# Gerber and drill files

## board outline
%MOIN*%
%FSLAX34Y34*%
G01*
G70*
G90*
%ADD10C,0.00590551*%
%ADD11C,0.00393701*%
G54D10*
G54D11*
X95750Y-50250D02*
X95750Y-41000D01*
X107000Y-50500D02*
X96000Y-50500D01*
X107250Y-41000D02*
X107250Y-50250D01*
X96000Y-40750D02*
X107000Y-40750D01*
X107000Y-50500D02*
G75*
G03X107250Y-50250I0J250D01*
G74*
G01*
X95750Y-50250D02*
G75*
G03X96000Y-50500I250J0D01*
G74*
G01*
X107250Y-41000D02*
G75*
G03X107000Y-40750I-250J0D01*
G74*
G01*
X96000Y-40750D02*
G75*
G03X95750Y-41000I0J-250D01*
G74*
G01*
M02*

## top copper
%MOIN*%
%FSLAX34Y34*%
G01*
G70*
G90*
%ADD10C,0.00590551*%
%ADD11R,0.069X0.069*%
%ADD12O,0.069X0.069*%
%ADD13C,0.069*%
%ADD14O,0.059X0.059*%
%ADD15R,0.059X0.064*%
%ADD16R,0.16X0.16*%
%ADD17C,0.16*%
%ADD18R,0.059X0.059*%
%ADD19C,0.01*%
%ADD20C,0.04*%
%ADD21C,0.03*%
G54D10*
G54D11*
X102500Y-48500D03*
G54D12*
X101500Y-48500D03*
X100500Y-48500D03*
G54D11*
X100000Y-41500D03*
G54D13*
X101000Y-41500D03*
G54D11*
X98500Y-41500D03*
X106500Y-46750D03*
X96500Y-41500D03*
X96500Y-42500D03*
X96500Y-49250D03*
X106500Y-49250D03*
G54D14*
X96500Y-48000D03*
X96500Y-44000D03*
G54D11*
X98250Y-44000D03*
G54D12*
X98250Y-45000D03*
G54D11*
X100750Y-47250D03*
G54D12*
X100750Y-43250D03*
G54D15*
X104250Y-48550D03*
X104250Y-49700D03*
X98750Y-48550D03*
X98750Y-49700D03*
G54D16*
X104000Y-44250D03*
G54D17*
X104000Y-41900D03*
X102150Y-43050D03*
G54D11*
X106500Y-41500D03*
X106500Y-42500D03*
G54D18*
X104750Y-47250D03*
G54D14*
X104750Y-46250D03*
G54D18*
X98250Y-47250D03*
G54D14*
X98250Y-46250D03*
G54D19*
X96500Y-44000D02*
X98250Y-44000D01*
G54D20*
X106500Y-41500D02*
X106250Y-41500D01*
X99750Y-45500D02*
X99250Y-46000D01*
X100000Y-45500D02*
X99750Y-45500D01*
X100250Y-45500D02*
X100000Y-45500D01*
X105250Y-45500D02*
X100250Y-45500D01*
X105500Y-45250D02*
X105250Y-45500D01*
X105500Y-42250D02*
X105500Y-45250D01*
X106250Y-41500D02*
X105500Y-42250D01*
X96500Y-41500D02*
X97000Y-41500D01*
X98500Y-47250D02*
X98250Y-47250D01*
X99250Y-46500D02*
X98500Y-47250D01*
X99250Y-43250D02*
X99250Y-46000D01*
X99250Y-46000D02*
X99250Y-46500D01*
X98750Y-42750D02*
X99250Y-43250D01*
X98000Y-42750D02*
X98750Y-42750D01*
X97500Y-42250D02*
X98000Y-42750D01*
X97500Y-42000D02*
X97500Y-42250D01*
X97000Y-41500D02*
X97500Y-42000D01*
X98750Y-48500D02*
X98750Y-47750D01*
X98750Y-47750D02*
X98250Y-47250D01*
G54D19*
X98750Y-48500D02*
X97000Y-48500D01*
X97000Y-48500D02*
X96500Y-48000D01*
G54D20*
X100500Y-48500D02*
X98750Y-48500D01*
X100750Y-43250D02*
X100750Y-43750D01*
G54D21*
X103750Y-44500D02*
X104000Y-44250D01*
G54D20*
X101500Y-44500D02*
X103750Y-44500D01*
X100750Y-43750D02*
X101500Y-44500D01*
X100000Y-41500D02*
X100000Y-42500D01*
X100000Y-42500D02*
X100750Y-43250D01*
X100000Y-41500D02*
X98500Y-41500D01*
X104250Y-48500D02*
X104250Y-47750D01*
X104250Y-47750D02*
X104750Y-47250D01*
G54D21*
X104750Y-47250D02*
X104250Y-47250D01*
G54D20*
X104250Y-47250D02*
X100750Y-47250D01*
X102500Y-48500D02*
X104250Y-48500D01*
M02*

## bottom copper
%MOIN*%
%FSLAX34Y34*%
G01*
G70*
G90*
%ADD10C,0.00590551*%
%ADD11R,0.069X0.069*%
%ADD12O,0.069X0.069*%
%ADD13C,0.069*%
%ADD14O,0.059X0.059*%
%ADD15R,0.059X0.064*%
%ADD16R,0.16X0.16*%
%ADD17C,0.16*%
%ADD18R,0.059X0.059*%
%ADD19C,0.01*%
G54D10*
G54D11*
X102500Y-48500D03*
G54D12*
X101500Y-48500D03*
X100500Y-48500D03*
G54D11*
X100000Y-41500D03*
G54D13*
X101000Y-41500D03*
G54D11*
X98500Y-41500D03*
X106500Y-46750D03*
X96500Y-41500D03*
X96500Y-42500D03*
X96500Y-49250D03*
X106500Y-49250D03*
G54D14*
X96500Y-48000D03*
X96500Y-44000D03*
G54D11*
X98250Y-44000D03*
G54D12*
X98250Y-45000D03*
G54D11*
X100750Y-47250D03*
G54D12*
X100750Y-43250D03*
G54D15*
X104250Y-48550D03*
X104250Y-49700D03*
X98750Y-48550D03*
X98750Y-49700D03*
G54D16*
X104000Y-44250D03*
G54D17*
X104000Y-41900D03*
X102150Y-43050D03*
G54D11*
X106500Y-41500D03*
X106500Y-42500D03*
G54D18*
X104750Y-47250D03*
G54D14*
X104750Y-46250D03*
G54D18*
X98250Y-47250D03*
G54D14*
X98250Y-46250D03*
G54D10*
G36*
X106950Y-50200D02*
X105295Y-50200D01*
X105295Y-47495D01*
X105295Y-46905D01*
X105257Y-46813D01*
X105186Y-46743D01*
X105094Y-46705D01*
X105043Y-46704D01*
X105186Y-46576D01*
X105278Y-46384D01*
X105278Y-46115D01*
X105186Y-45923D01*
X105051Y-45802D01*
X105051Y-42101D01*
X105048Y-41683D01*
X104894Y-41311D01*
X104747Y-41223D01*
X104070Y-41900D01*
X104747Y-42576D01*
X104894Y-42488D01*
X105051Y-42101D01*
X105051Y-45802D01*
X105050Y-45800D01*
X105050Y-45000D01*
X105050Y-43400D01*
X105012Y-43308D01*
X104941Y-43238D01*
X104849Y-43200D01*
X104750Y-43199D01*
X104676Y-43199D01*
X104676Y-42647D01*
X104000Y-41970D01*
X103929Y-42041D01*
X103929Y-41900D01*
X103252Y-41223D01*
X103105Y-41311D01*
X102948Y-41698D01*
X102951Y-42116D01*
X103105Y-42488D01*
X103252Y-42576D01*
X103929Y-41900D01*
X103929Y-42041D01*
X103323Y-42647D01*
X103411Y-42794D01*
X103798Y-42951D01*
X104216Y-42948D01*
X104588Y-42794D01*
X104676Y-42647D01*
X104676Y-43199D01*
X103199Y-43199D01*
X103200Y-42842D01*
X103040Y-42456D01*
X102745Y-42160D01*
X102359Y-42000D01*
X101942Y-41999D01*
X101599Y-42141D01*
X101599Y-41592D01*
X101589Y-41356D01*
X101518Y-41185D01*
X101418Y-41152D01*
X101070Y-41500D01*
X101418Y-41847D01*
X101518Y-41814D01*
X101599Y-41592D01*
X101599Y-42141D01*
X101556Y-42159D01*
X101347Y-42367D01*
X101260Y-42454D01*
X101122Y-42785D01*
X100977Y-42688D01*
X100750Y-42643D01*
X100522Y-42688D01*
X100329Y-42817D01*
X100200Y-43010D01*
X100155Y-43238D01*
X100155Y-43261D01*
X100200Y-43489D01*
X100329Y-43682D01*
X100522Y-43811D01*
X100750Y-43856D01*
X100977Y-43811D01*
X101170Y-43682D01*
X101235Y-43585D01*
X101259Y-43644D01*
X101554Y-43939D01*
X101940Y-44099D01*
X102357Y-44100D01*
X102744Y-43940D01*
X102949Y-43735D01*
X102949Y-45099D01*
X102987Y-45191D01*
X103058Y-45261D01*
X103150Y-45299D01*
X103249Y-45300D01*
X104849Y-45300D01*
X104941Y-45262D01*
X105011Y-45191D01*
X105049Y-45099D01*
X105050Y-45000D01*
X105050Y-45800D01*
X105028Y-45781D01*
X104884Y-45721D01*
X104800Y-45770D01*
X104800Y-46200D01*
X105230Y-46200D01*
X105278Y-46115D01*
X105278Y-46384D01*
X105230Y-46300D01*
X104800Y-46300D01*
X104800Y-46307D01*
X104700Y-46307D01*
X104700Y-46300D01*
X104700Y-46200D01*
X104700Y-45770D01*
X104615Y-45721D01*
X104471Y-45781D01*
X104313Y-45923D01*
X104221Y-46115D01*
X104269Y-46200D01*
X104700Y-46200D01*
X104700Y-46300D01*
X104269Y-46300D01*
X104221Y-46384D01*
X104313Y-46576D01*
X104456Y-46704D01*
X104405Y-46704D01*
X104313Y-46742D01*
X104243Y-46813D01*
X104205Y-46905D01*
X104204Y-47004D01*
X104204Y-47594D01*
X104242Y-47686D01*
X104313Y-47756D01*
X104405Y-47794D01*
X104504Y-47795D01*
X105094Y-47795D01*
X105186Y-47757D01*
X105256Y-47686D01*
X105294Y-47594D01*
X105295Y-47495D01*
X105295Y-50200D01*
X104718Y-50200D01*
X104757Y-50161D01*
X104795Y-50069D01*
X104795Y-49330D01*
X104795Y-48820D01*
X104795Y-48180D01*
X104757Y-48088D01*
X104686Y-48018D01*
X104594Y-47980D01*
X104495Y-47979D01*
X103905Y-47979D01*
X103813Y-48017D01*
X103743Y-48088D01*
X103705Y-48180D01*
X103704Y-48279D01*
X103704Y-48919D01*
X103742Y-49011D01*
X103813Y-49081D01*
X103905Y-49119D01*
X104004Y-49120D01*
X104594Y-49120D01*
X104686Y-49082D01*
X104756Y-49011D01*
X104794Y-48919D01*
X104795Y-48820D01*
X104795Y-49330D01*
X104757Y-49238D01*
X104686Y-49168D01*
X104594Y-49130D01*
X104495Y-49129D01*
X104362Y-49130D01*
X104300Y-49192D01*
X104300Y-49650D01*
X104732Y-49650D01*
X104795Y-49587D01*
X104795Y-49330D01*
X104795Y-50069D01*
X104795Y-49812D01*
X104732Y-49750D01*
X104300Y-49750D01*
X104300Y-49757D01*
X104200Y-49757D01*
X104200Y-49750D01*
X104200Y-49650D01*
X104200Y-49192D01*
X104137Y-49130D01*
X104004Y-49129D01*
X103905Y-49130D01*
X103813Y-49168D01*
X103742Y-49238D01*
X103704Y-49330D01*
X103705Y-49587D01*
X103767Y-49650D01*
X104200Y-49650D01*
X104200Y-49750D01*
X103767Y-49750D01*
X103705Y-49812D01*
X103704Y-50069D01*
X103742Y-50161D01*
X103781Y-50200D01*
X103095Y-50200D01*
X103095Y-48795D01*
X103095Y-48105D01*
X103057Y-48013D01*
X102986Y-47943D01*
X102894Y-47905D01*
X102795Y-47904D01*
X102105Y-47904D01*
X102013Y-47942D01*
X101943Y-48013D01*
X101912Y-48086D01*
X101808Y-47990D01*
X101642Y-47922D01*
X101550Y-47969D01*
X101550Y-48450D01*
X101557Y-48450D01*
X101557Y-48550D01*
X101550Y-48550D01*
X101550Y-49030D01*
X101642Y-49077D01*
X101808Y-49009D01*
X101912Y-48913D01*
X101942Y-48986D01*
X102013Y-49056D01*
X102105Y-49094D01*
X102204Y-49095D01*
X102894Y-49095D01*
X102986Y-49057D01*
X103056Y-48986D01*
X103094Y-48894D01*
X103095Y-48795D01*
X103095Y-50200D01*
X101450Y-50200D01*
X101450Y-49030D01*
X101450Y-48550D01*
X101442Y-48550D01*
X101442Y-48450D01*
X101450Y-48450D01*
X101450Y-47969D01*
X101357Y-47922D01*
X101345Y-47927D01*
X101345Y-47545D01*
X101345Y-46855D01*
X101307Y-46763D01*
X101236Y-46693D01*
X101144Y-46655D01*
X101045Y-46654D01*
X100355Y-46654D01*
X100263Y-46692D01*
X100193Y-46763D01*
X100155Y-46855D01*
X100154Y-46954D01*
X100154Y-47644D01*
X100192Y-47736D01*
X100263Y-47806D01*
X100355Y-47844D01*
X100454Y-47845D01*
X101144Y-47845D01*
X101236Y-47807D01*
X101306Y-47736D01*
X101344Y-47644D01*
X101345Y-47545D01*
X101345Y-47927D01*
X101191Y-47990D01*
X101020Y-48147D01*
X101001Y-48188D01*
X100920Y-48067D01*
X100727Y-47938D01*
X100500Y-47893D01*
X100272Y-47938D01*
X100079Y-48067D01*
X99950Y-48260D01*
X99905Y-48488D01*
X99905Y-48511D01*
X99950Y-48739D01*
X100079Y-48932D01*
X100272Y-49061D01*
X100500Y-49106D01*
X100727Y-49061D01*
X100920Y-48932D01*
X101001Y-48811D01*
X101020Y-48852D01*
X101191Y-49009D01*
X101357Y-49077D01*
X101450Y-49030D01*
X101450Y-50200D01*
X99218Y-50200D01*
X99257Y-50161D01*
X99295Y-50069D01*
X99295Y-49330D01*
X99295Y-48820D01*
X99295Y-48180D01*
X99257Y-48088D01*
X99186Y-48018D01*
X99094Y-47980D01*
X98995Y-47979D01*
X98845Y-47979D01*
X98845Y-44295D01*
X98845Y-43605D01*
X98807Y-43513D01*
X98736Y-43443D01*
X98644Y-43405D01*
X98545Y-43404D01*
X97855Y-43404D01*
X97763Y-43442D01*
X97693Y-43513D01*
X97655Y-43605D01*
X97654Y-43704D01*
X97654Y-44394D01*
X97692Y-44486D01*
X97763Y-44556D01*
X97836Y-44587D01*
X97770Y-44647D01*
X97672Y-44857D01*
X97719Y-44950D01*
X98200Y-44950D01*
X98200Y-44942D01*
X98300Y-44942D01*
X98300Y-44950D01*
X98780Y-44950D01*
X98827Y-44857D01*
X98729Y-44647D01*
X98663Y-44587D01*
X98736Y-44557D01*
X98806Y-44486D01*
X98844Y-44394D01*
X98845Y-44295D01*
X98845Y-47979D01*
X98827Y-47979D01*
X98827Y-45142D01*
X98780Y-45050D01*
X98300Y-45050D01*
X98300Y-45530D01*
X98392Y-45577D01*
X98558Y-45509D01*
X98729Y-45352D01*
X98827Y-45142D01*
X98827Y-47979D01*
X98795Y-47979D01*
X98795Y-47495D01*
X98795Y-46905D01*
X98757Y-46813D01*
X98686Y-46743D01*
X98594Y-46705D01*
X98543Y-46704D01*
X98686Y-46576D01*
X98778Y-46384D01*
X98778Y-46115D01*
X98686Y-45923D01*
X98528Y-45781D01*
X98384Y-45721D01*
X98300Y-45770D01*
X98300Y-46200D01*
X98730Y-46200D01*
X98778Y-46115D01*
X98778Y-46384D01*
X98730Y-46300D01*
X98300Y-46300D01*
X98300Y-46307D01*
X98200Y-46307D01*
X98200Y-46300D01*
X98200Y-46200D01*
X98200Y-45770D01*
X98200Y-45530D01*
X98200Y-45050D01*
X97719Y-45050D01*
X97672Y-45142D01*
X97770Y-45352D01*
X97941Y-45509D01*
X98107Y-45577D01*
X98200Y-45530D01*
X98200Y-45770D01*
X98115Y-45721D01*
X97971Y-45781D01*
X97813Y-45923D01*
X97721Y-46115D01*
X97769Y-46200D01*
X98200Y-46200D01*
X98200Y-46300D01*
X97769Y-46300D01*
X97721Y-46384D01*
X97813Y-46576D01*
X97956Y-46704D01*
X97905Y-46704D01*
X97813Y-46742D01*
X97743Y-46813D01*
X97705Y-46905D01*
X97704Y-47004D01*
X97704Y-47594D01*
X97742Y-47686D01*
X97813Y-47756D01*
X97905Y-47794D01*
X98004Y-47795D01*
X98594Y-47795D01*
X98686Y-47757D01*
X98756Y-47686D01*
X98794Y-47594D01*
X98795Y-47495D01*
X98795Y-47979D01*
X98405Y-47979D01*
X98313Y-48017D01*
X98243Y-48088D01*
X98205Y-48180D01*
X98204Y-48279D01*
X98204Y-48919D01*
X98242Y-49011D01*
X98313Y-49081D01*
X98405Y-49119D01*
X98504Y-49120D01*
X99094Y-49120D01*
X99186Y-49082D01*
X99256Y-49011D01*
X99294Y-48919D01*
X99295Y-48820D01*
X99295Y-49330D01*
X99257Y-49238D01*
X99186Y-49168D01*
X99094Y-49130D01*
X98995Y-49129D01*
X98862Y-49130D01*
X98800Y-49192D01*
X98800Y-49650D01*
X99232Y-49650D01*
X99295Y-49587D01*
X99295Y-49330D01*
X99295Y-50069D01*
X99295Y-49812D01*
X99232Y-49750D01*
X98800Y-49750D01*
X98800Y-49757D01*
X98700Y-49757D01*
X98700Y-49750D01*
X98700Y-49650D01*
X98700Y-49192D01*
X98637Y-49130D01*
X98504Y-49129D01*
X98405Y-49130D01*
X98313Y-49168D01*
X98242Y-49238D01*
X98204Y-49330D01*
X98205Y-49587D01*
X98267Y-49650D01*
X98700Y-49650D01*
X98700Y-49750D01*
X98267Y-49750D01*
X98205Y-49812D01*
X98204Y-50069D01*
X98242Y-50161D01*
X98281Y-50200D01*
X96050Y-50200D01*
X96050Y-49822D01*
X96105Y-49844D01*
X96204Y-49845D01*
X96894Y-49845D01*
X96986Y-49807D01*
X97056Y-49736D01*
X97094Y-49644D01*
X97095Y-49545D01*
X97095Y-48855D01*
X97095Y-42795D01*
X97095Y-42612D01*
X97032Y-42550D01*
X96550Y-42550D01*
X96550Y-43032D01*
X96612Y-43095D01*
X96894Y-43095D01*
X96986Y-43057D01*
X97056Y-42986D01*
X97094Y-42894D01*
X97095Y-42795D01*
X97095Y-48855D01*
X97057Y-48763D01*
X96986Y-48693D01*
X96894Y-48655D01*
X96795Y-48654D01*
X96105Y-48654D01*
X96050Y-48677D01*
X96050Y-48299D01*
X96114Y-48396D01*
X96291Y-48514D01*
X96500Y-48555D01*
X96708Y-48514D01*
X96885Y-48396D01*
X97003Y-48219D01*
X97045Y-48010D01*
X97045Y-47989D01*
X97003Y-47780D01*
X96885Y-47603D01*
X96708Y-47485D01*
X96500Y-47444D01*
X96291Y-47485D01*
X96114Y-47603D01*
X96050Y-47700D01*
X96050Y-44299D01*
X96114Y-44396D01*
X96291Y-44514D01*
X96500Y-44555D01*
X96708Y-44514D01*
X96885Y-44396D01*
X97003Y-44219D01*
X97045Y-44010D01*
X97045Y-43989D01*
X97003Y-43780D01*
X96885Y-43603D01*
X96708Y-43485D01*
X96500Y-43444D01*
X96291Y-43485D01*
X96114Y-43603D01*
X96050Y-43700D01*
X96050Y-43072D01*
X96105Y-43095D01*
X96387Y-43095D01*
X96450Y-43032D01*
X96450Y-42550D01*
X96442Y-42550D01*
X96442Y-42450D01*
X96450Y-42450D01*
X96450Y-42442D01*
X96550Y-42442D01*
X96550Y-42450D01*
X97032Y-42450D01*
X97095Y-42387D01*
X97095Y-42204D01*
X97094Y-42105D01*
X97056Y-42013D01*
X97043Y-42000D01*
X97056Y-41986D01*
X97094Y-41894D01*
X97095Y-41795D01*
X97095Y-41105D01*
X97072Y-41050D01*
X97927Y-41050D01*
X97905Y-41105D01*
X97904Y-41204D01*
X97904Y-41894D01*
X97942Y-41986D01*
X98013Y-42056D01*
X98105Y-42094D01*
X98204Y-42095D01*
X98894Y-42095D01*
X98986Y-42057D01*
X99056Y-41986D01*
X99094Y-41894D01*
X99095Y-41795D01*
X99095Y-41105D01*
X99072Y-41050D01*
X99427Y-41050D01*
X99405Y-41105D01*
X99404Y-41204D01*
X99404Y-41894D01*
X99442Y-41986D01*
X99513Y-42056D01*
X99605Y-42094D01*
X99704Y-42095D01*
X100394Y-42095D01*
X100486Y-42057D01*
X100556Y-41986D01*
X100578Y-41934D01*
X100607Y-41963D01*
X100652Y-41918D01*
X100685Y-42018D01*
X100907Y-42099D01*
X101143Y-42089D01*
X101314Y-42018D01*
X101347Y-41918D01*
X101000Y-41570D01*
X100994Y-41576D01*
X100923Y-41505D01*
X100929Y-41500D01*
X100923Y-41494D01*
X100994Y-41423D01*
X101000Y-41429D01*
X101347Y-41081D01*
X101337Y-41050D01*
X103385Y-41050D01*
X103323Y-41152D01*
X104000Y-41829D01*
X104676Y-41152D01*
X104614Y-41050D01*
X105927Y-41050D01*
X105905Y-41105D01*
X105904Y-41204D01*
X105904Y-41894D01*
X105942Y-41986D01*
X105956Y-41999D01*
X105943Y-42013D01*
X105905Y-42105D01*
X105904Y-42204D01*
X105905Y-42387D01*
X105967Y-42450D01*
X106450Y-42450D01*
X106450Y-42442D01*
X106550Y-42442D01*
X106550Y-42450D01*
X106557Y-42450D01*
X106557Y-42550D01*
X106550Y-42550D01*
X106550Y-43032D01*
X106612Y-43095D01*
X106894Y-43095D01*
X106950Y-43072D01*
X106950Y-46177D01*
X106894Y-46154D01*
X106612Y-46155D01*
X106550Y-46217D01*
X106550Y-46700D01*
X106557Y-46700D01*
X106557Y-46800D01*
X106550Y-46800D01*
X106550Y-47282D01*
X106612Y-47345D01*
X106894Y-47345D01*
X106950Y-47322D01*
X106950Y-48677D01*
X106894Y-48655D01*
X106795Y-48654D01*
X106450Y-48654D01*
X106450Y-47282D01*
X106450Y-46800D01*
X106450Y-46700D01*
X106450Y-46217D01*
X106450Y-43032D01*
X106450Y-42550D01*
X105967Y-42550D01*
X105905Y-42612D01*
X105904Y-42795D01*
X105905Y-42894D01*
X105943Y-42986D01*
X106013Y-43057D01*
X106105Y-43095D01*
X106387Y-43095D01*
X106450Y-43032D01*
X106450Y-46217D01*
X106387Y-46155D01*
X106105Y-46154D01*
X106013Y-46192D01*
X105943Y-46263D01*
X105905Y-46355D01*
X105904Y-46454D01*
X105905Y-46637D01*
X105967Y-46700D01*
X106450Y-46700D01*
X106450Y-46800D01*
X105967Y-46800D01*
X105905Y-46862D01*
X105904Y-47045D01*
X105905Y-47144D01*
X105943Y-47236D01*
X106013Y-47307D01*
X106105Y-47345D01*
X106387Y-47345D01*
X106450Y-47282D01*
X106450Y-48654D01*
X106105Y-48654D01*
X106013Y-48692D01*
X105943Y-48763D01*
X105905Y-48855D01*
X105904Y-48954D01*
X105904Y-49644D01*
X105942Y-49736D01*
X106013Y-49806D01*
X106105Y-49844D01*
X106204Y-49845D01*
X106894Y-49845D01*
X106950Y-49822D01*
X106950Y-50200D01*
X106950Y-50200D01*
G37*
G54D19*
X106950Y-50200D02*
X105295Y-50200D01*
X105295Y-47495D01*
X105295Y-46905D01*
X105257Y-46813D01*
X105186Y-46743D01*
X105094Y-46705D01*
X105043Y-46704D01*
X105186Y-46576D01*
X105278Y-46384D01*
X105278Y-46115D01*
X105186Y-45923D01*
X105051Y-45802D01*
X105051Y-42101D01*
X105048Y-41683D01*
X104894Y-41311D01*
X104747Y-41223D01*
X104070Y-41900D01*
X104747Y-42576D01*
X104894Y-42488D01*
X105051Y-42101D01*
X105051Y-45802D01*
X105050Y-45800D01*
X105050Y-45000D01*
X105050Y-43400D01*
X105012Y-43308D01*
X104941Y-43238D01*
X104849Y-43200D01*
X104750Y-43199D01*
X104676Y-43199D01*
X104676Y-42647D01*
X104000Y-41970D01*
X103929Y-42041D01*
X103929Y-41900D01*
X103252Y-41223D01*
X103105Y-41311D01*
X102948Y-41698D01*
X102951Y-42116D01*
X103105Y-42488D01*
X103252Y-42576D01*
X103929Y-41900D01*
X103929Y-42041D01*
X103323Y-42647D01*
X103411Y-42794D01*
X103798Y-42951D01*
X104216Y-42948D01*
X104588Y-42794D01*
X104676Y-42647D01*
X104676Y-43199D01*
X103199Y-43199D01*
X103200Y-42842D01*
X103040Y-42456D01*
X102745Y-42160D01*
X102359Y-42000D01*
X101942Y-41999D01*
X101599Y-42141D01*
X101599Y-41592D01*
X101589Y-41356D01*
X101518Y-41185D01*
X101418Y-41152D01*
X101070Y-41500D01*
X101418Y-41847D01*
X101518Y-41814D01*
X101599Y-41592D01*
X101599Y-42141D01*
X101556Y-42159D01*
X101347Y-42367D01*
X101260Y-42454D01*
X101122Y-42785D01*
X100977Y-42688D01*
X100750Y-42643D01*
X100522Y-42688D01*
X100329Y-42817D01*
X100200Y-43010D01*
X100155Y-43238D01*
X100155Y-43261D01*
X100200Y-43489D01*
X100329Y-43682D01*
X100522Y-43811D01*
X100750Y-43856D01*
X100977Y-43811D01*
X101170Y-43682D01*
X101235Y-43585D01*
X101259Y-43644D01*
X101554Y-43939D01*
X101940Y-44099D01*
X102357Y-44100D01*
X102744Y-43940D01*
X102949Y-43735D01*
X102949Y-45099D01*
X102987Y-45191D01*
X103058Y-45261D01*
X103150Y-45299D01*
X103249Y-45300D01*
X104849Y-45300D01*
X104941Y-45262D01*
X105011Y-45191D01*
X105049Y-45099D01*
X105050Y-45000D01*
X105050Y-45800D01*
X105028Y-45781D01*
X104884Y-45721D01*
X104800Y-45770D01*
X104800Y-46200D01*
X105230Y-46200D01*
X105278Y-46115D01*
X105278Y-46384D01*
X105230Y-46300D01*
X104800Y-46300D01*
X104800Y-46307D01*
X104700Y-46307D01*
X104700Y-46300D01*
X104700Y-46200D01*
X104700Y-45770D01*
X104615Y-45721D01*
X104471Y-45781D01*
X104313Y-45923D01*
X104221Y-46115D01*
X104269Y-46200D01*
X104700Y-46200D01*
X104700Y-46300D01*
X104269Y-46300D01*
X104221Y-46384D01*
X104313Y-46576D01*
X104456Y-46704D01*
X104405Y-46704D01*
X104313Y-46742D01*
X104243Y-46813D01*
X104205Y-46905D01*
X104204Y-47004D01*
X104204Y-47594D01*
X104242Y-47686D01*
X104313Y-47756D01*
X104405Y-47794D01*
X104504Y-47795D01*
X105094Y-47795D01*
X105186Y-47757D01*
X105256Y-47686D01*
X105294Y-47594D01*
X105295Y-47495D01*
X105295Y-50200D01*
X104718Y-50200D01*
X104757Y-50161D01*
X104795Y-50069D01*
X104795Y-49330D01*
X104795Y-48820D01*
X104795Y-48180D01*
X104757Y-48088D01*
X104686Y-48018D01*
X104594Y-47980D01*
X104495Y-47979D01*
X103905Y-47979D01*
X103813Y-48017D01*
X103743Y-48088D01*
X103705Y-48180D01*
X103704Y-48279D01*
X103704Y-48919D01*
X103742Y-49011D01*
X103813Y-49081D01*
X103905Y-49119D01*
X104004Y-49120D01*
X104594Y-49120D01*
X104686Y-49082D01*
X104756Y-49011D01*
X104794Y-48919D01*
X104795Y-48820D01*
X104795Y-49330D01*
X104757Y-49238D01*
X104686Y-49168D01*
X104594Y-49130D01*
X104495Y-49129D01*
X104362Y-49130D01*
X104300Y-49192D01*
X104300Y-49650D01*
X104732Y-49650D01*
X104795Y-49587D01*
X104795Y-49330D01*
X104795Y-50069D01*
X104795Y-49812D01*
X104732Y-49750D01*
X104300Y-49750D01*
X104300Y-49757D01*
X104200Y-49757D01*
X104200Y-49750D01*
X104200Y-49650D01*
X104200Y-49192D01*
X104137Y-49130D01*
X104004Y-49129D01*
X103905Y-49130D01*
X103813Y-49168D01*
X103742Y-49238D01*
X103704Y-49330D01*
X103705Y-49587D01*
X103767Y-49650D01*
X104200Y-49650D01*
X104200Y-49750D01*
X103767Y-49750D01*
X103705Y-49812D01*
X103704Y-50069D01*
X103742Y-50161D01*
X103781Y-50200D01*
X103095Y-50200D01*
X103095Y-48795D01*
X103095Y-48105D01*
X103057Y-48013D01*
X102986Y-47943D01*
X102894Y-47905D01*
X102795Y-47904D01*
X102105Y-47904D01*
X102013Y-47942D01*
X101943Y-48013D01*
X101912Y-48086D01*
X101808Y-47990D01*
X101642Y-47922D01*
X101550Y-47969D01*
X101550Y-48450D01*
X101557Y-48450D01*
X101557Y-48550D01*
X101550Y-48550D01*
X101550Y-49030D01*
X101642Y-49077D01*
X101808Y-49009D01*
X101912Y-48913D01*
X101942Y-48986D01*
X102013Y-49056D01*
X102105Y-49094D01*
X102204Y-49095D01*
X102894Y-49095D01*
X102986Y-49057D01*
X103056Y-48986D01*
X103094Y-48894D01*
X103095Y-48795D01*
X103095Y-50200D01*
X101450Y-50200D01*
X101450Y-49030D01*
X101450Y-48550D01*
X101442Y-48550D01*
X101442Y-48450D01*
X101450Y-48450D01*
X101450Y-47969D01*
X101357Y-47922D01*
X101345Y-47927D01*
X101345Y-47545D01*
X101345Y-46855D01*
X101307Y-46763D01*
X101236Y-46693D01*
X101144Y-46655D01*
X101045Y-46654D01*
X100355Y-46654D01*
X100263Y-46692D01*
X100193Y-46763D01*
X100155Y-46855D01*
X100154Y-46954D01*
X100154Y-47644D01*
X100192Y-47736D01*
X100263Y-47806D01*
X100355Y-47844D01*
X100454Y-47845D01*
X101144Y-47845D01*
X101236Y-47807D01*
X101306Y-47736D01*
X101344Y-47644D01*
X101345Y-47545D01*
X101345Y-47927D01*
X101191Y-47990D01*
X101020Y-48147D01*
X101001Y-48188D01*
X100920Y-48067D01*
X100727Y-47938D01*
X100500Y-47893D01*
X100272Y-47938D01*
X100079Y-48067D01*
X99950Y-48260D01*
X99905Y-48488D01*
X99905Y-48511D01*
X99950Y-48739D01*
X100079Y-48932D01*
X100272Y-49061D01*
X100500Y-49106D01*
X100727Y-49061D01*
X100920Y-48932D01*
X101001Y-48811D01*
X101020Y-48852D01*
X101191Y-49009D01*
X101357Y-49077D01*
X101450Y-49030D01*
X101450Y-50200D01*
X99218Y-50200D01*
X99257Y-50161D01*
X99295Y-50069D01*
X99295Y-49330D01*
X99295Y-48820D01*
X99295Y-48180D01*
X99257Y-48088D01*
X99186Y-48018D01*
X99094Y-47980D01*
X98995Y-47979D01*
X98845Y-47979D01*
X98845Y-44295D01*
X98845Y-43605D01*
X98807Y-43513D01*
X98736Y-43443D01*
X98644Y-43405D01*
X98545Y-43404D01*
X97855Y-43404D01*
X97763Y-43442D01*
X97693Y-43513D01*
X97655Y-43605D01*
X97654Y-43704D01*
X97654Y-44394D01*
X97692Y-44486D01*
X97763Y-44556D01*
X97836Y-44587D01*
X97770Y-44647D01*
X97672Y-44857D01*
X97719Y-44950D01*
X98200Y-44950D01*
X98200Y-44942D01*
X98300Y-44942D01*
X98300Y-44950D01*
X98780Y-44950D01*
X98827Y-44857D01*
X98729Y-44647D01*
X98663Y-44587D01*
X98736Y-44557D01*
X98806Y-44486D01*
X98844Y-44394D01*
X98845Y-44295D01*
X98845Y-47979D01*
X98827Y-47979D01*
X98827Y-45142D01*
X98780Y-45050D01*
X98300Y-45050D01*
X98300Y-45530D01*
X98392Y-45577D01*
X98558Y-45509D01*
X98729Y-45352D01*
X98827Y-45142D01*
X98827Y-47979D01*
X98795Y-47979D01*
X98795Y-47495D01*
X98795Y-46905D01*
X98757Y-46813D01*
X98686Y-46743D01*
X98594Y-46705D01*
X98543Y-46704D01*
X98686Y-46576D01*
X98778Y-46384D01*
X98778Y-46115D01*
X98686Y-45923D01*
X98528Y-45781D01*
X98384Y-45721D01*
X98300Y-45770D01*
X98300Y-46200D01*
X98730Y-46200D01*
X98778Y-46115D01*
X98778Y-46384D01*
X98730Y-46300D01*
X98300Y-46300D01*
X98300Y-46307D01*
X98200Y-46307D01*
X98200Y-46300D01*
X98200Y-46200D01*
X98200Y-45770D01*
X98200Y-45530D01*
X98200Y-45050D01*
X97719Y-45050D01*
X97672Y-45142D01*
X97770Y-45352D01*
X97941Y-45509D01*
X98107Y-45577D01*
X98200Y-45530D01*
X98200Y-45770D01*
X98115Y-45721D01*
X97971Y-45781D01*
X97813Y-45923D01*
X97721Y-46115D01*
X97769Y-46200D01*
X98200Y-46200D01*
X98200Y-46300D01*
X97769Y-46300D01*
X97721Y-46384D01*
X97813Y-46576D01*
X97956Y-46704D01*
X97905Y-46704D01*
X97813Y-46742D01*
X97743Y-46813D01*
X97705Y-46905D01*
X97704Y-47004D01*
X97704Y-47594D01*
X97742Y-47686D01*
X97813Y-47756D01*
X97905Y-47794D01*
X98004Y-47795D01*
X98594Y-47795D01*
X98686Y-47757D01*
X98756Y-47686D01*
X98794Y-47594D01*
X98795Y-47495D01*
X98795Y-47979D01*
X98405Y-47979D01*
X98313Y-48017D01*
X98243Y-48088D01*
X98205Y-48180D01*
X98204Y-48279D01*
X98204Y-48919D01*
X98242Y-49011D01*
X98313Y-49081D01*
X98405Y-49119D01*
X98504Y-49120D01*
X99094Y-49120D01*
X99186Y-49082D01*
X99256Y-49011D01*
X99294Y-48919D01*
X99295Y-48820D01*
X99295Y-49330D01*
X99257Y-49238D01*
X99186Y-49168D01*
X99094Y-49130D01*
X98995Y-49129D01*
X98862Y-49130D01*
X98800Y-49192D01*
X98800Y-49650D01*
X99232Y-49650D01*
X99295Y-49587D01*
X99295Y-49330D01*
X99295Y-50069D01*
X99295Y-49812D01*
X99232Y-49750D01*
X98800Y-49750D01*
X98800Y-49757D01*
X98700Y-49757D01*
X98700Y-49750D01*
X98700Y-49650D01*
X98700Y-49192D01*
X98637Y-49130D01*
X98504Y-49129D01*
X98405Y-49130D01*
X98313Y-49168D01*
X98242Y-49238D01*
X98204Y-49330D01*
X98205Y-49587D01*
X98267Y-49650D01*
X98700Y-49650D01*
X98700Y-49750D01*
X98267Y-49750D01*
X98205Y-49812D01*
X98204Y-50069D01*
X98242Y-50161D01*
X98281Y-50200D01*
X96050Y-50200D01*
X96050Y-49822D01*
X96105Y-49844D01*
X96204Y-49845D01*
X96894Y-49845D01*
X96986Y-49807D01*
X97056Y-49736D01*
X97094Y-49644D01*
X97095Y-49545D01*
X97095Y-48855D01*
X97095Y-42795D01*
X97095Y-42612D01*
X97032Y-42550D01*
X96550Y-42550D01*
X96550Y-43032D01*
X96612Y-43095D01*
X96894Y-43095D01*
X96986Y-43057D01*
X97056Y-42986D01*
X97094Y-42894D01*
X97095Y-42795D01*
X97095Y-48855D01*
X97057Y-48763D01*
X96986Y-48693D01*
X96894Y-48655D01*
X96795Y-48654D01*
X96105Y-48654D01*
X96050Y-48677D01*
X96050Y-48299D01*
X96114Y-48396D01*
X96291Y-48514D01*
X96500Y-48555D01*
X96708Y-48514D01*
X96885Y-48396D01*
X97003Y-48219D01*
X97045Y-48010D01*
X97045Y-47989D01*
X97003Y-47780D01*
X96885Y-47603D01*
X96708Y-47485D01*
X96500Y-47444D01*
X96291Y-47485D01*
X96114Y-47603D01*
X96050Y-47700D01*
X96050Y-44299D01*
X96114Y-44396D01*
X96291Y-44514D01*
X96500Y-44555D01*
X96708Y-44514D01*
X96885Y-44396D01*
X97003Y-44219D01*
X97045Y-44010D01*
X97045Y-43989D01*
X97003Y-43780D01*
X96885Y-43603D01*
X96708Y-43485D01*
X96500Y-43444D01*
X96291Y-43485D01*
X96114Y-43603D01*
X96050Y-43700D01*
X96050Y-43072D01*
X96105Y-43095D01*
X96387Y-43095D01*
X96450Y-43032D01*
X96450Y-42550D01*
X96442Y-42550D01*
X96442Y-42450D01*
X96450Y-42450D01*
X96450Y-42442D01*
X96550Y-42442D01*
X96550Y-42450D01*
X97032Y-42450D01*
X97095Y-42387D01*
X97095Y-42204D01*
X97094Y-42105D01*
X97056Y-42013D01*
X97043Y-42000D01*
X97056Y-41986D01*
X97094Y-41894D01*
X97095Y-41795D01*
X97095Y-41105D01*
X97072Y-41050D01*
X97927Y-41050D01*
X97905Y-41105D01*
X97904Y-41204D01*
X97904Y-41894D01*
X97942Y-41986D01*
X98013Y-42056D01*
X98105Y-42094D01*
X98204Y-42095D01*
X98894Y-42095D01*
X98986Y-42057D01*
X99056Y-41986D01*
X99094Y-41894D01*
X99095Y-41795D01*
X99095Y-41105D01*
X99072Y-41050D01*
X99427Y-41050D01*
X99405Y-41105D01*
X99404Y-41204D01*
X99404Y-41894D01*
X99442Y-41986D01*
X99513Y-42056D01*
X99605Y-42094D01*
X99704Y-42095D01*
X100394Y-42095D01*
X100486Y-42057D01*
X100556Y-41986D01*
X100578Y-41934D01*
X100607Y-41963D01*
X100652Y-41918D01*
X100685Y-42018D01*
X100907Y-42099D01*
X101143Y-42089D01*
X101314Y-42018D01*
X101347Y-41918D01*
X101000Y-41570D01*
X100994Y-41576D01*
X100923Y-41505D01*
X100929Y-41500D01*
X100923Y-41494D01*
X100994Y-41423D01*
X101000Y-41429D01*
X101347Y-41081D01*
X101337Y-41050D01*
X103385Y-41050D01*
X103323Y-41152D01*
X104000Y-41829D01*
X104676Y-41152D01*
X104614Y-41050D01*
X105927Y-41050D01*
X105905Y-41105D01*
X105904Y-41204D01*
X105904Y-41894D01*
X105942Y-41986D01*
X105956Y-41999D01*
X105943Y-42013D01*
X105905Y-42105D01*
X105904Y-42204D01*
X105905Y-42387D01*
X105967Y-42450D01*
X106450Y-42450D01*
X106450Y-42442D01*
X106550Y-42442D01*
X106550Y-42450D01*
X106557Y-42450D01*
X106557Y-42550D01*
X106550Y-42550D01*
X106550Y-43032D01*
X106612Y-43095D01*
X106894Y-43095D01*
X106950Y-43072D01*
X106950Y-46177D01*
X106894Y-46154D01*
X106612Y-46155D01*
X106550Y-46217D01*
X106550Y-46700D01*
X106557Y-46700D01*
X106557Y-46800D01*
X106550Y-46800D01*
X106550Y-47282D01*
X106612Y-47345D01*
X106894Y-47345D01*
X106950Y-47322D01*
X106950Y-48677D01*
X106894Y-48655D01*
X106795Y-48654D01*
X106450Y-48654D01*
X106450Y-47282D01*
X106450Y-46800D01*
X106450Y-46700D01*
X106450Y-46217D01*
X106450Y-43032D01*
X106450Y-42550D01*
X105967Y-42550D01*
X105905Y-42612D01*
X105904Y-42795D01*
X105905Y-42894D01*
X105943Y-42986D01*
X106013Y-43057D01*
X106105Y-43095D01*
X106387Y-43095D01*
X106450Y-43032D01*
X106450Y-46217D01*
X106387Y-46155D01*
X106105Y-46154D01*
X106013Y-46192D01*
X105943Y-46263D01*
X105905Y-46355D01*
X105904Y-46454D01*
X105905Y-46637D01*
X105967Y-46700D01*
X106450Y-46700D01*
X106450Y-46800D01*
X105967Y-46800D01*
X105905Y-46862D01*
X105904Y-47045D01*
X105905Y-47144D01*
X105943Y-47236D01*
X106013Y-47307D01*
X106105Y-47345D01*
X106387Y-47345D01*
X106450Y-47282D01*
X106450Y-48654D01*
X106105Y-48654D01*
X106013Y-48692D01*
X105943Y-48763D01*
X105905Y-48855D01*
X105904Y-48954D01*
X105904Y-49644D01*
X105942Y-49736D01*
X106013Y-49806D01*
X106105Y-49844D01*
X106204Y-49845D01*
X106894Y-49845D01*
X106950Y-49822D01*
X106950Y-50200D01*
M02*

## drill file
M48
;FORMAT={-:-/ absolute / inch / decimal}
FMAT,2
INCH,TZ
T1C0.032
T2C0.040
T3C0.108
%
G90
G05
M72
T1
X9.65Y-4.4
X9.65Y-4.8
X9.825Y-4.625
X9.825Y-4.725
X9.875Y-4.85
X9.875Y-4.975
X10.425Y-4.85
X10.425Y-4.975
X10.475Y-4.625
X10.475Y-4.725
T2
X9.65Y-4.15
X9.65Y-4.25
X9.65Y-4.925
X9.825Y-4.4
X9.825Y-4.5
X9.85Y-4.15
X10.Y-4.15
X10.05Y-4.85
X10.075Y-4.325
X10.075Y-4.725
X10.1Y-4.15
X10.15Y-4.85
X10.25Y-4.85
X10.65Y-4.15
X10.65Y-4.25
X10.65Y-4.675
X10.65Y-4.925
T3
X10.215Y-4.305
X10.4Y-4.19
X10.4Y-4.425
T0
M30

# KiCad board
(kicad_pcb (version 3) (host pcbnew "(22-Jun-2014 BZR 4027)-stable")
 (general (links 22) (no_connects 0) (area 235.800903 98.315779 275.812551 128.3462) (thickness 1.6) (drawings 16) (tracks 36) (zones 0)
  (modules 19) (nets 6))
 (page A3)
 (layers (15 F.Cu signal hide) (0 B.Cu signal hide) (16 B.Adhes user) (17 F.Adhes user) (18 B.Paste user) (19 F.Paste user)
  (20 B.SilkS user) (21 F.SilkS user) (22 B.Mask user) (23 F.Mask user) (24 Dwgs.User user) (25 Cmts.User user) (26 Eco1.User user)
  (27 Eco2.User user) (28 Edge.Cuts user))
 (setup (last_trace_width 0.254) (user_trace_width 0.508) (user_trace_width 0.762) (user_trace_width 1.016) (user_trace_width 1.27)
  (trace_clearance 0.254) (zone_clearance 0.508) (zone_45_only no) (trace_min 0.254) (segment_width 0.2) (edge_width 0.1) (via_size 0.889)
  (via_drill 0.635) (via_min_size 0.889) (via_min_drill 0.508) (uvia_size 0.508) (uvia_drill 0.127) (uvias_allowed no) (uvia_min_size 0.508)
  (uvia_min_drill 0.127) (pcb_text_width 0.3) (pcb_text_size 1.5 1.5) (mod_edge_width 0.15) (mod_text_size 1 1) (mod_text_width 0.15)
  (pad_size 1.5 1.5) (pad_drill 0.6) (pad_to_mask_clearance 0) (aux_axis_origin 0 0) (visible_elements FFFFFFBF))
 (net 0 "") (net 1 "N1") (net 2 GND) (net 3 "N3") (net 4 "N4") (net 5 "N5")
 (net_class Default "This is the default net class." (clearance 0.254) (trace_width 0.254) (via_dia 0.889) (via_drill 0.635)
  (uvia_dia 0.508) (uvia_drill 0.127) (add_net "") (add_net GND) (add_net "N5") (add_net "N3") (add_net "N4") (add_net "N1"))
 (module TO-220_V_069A (layer F.Cu) (at 260.35 123.19 180)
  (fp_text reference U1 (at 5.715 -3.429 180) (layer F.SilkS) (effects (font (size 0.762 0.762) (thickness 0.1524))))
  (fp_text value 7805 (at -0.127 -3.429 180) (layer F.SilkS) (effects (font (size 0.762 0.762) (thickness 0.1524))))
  (pad 1 thru_hole rect (at 0 0 270) (size 1.7526 1.7526) (drill 1.016) (layers *.Cu *.Mask F.SilkS) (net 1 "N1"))
  (pad 2 thru_hole oval (at 2.54 0 270) (size 1.7526 1.7526) (drill 1.016) (layers *.Cu *.Mask F.SilkS) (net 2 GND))
  (pad 3 thru_hole oval (at 5.08 0 270) (size 1.7526 1.7526) (drill 1.016) (layers *.Cu *.Mask F.SilkS) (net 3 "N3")))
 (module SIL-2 (layer F.Cu) (at 254 105.41)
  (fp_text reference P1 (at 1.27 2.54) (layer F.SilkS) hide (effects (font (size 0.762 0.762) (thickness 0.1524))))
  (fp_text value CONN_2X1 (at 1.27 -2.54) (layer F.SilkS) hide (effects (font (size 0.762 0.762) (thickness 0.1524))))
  (pad 1 thru_hole rect (at 0 0) (size 1.7526 1.7526) (drill 1.016) (layers *.Cu *.Mask F.SilkS) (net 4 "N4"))
  (pad 2 thru_hole circle (at 2.54 0) (size 1.7526 1.7526) (drill 1.016) (layers *.Cu *.Mask F.SilkS) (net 2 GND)))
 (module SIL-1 (layer F.Cu) (at 250.19 105.41)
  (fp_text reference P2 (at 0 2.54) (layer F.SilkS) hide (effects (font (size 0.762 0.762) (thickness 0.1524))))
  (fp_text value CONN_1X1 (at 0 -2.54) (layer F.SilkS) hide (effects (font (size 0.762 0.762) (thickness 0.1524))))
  (pad 1 thru_hole rect (at 0 0) (size 1.7526 1.7526) (drill 1.016) (layers *.Cu *.Mask F.SilkS) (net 4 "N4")))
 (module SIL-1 (layer F.Cu) (at 270.51 118.745)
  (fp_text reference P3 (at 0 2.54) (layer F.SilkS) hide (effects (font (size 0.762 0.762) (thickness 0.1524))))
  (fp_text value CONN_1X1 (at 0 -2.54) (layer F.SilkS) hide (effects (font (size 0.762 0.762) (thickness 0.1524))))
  (pad 1 thru_hole rect (at 0 0) (size 1.7526 1.7526) (drill 1.016) (layers *.Cu *.Mask F.SilkS) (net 2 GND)))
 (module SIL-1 (layer F.Cu) (at 245.11 105.41)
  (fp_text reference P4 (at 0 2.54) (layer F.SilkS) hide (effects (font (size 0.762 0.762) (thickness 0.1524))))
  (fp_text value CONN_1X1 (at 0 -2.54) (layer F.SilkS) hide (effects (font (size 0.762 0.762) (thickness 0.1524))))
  (pad 1 thru_hole rect (at 0 0) (size 1.7526 1.7526) (drill 1.016) (layers *.Cu *.Mask F.SilkS) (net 3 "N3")))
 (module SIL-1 (layer F.Cu) (at 245.11 107.95)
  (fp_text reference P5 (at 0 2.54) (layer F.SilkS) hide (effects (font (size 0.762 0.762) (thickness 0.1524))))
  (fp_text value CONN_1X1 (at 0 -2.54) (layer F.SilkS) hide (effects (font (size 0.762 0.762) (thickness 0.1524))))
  (pad 1 thru_hole rect (at 0 0) (size 1.7526 1.7526) (drill 1.016) (layers *.Cu *.Mask F.SilkS) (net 2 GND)))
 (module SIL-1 (layer F.Cu) (at 245.11 125.095)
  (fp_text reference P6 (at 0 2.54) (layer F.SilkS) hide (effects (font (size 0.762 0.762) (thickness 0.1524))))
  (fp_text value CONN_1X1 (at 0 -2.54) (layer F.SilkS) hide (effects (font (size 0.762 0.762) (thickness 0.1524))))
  (pad 1 thru_hole rect (at 0 0) (size 1.7526 1.7526) (drill 1.016) (layers *.Cu *.Mask F.SilkS)))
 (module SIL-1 (layer F.Cu) (at 270.51 125.095)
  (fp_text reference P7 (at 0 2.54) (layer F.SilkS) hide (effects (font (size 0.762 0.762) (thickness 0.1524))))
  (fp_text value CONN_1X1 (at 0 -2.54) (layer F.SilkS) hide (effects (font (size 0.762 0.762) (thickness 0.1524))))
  (pad 1 thru_hole rect (at 0 0) (size 1.7526 1.7526) (drill 1.016) (layers *.Cu *.Mask F.SilkS)))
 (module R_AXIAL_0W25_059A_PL (layer F.Cu) (at 245.11 121.92 90) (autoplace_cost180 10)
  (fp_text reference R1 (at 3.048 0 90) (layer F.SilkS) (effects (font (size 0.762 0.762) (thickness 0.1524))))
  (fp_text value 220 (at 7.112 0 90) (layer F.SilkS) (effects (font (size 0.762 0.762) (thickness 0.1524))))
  (pad 1 thru_hole oval (at 0 0 90) (size 1.4986 1.4986) (drill 0.8128) (layers *.Cu *.Mask F.SilkS) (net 3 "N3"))
  (pad 2 thru_hole oval (at 10.16 0 90) (size 1.4986 1.4986) (drill 0.8128) (layers *.Cu *.Mask F.SilkS) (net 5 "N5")))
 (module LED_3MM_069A (layer F.Cu) (at 249.555 111.76 270)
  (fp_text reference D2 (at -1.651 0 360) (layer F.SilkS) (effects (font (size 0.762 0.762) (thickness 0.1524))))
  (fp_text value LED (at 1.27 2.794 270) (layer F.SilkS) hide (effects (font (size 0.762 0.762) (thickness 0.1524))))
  (pad 1 thru_hole rect (at 0 0 270) (size 1.7526 1.7526) (drill 1.016) (layers *.Cu *.Mask F.SilkS) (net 5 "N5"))
  (pad 2 thru_hole oval (at 2.54 0 270) (size 1.7526 1.7526) (drill 1.016) (layers *.Cu *.Mask F.SilkS) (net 2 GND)))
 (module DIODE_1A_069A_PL (layer F.Cu) (at 255.905 114.935 270)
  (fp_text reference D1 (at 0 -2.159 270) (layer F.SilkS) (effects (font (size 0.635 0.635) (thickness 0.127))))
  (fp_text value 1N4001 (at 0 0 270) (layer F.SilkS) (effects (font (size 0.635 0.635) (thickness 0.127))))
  (pad 2 thru_hole rect (at 5.08 0 270) (size 1.7526 1.7526) (drill 1.016) (layers *.Cu *.Mask F.SilkS) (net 1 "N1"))
  (pad 1 thru_hole oval (at -5.08 0 270) (size 1.7526 1.7526) (drill 1.016) (layers *.Cu *.Mask F.SilkS) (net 4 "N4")))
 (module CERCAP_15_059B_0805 (layer F.Cu) (at 264.795 123.19 270)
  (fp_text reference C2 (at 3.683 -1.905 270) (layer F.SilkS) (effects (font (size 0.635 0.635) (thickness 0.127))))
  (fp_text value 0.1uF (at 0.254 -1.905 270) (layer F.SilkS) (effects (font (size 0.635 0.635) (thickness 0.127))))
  (pad 1 thru_hole rect (at 0 0 270) (size 1.6256 1.4986) (drill 0.8128 (offset 0.127 0)) (layers *.Cu *.Mask F.SilkS) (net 1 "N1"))
  (pad 2 thru_hole rect (at 3.175 0 270) (size 1.6256 1.4986) (drill 0.8128 (offset -0.127 0)) (layers *.Cu *.Mask F.SilkS) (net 2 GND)))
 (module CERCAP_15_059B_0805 (layer F.Cu) (at 250.825 123.19 270)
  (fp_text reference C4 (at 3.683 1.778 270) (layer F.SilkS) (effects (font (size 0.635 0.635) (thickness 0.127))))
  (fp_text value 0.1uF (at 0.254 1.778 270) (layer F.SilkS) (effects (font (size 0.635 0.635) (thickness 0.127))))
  (pad 1 thru_hole rect (at 0 0 270) (size 1.6256 1.4986) (drill 0.8128 (offset 0.127 0)) (layers *.Cu *.Mask F.SilkS) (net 3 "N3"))
  (pad 2 thru_hole rect (at 3.175 0 270) (size 1.6256 1.4986) (drill 0.8128 (offset -0.127 0)) (layers *.Cu *.Mask F.SilkS) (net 2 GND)))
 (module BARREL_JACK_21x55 (layer F.Cu) (at 264.16 112.395 270)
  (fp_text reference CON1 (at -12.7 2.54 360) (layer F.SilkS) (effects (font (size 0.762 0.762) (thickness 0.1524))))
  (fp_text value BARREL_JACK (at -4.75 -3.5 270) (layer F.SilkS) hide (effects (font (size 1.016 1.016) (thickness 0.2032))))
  (pad 1 thru_hole rect (at 0 0 270) (size 4.064 4.064) (drill 2.7432) (layers *.Cu *.Mask F.SilkS) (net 4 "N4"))
  (pad 2 thru_hole circle (at -5.969 0 270) (size 4.064 4.064) (drill 2.7432) (layers *.Cu *.Mask F.SilkS) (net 2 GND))
  (pad 3 thru_hole circle (at -3.048 4.699 270) (size 4.064 4.064) (drill 2.7432) (layers *.Cu *.Mask F.SilkS)))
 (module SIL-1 (layer F.Cu) (at 270.51 105.41)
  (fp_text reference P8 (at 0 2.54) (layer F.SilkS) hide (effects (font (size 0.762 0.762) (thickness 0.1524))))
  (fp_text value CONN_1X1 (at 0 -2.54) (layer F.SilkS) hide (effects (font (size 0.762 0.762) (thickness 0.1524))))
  (pad 1 thru_hole rect (at 0 0) (size 1.7526 1.7526) (drill 1.016) (layers *.Cu *.Mask F.SilkS) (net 3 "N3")))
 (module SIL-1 (layer F.Cu) (at 270.51 107.95)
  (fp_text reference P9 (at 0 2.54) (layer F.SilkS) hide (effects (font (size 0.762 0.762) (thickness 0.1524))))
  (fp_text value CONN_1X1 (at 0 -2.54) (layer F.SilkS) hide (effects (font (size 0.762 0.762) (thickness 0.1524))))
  (pad 1 thru_hole rect (at 0 0) (size 1.7526 1.7526) (drill 1.016) (layers *.Cu *.Mask F.SilkS) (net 2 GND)))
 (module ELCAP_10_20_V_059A (layer F.Cu) (at 266.065 120.015 90)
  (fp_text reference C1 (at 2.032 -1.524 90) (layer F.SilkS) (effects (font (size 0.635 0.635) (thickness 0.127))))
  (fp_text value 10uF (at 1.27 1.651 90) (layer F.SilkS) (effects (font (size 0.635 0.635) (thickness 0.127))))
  (pad 1 thru_hole rect (at 0 0 90) (size 1.4986 1.4986) (drill 0.8128) (layers *.Cu *.Mask F.SilkS) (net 1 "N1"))
  (pad 2 thru_hole oval (at 2.54 0 90) (size 1.4986 1.4986) (drill 0.8128) (layers *.Cu *.Mask F.SilkS) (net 2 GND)))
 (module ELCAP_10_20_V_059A (layer F.Cu) (at 249.555 120.015 90)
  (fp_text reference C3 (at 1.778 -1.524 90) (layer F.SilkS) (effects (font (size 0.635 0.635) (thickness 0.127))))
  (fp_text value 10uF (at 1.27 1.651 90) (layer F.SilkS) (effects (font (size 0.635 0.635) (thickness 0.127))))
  (pad 1 thru_hole rect (at 0 0 90) (size 1.4986 1.4986) (drill 0.8128) (layers *.Cu *.Mask F.SilkS) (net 3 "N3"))
  (pad 2 thru_hole oval (at 2.54 0 90) (size 1.4986 1.4986) (drill 0.8128) (layers *.Cu *.Mask F.SilkS) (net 2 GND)))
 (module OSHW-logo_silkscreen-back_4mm (layer F.Cu) (at 257.81 116.205 270)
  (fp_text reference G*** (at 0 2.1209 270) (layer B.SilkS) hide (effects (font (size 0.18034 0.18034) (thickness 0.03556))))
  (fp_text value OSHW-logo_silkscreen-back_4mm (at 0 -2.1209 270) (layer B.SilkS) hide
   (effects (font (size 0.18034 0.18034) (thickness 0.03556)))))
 (gr_line (start 243.205 127.635) (end 243.205 104.14) (angle 90) (layer Edge.Cuts) (width 0.1))
 (gr_line (start 271.78 128.27) (end 243.84 128.27) (angle 90) (layer Edge.Cuts) (width 0.1))
 (gr_line (start 272.415 104.14) (end 272.415 127.635) (angle 90) (layer Edge.Cuts) (width 0.1))
 (gr_line (start 243.84 103.505) (end 271.78 103.505) (angle 90) (layer Edge.Cuts) (width 0.1))
 (gr_arc (start 271.78 127.635) (end 272.415 127.635) (angle 90) (layer Edge.Cuts) (width 0.1))
 (gr_arc (start 243.84 127.635) (end 243.84 128.27) (angle 90) (layer Edge.Cuts) (width 0.1))
 (gr_arc (start 271.78 104.14) (end 271.78 103.505) (angle 90) (layer Edge.Cuts) (width 0.1))
 (gr_arc (start 243.84 104.14) (end 243.205 104.14) (angle 90) (layer Edge.Cuts) (width 0.1))
 (segment (start 245.11 111.76) (end 249.555 111.76) (width 0.254) (layer F.Cu) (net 5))
 (segment (start 270.51 105.41) (end 269.875 105.41) (width 1.016) (layer F.Cu) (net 3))
 (segment (start 253.365 115.57) (end 252.095 116.84) (width 1.016) (layer F.Cu) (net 3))
 (segment (start 254 115.57) (end 253.365 115.57) (width 1.016) (layer F.Cu) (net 3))
 (segment (start 254.635 115.57) (end 254 115.57) (width 1.016) (layer F.Cu) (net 3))
 (segment (start 267.335 115.57) (end 254.635 115.57) (width 1.016) (layer F.Cu) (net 3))
 (segment (start 267.97 114.935) (end 267.335 115.57) (width 1.016) (layer F.Cu) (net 3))
 (segment (start 267.97 107.315) (end 267.97 114.935) (width 1.016) (layer F.Cu) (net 3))
 (segment (start 269.875 105.41) (end 267.97 107.315) (width 1.016) (layer F.Cu) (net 3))
 (segment (start 245.11 105.41) (end 246.38 105.41) (width 1.016) (layer F.Cu) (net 3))
 (segment (start 250.19 120.015) (end 249.555 120.015) (width 1.016) (layer F.Cu) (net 3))
 (segment (start 252.095 118.11) (end 250.19 120.015) (width 1.016) (layer F.Cu) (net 3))
 (segment (start 252.095 109.855) (end 252.095 116.84) (width 1.016) (layer F.Cu) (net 3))
 (segment (start 252.095 116.84) (end 252.095 118.11) (width 1.016) (layer F.Cu) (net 3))
 (segment (start 250.825 108.585) (end 252.095 109.855) (width 1.016) (layer F.Cu) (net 3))
 (segment (start 248.92 108.585) (end 250.825 108.585) (width 1.016) (layer F.Cu) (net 3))
 (segment (start 247.65 107.315) (end 248.92 108.585) (width 1.016) (layer F.Cu) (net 3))
 (segment (start 247.65 106.68) (end 247.65 107.315) (width 1.016) (layer F.Cu) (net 3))
 (segment (start 246.38 105.41) (end 247.65 106.68) (width 1.016) (layer F.Cu) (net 3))
 (segment (start 250.825 123.19) (end 250.825 121.285) (width 1.016) (layer F.Cu) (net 3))
 (segment (start 250.825 121.285) (end 249.555 120.015) (width 1.016) (layer F.Cu) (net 3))
 (segment (start 250.825 123.19) (end 246.38 123.19) (width 0.254) (layer F.Cu) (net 3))
 (segment (start 246.38 123.19) (end 245.11 121.92) (width 0.254) (layer F.Cu) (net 3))
 (segment (start 255.27 123.19) (end 250.825 123.19) (width 1.016) (layer F.Cu) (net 3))
 (segment (start 255.905 109.855) (end 255.905 111.125) (width 1.016) (layer F.Cu) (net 4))
 (segment (start 263.525 113.03) (end 264.16 112.395) (width 0.762) (layer F.Cu) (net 4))
 (segment (start 257.81 113.03) (end 263.525 113.03) (width 1.016) (layer F.Cu) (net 4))
 (segment (start 255.905 111.125) (end 257.81 113.03) (width 1.016) (layer F.Cu) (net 4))
 (segment (start 254 105.41) (end 254 107.95) (width 1.016) (layer F.Cu) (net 4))
 (segment (start 254 107.95) (end 255.905 109.855) (width 1.016) (layer F.Cu) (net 4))
 (segment (start 254 105.41) (end 250.19 105.41) (width 1.016) (layer F.Cu) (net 4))
 (segment (start 264.795 123.19) (end 264.795 121.285) (width 1.016) (layer F.Cu) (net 1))
 (segment (start 264.795 121.285) (end 266.065 120.015) (width 1.016) (layer F.Cu) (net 1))
 (segment (start 266.065 120.015) (end 264.795 120.015) (width 0.762) (layer F.Cu) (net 1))
 (segment (start 264.795 120.015) (end 255.905 120.015) (width 1.016) (layer F.Cu) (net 1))
 (segment (start 260.35 123.19) (end 264.795 123.19) (width 1.016) (layer F.Cu) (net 1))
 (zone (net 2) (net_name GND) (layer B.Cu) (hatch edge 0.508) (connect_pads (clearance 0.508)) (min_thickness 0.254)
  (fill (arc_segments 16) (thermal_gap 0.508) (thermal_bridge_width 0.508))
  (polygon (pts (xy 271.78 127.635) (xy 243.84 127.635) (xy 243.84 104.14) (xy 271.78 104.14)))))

